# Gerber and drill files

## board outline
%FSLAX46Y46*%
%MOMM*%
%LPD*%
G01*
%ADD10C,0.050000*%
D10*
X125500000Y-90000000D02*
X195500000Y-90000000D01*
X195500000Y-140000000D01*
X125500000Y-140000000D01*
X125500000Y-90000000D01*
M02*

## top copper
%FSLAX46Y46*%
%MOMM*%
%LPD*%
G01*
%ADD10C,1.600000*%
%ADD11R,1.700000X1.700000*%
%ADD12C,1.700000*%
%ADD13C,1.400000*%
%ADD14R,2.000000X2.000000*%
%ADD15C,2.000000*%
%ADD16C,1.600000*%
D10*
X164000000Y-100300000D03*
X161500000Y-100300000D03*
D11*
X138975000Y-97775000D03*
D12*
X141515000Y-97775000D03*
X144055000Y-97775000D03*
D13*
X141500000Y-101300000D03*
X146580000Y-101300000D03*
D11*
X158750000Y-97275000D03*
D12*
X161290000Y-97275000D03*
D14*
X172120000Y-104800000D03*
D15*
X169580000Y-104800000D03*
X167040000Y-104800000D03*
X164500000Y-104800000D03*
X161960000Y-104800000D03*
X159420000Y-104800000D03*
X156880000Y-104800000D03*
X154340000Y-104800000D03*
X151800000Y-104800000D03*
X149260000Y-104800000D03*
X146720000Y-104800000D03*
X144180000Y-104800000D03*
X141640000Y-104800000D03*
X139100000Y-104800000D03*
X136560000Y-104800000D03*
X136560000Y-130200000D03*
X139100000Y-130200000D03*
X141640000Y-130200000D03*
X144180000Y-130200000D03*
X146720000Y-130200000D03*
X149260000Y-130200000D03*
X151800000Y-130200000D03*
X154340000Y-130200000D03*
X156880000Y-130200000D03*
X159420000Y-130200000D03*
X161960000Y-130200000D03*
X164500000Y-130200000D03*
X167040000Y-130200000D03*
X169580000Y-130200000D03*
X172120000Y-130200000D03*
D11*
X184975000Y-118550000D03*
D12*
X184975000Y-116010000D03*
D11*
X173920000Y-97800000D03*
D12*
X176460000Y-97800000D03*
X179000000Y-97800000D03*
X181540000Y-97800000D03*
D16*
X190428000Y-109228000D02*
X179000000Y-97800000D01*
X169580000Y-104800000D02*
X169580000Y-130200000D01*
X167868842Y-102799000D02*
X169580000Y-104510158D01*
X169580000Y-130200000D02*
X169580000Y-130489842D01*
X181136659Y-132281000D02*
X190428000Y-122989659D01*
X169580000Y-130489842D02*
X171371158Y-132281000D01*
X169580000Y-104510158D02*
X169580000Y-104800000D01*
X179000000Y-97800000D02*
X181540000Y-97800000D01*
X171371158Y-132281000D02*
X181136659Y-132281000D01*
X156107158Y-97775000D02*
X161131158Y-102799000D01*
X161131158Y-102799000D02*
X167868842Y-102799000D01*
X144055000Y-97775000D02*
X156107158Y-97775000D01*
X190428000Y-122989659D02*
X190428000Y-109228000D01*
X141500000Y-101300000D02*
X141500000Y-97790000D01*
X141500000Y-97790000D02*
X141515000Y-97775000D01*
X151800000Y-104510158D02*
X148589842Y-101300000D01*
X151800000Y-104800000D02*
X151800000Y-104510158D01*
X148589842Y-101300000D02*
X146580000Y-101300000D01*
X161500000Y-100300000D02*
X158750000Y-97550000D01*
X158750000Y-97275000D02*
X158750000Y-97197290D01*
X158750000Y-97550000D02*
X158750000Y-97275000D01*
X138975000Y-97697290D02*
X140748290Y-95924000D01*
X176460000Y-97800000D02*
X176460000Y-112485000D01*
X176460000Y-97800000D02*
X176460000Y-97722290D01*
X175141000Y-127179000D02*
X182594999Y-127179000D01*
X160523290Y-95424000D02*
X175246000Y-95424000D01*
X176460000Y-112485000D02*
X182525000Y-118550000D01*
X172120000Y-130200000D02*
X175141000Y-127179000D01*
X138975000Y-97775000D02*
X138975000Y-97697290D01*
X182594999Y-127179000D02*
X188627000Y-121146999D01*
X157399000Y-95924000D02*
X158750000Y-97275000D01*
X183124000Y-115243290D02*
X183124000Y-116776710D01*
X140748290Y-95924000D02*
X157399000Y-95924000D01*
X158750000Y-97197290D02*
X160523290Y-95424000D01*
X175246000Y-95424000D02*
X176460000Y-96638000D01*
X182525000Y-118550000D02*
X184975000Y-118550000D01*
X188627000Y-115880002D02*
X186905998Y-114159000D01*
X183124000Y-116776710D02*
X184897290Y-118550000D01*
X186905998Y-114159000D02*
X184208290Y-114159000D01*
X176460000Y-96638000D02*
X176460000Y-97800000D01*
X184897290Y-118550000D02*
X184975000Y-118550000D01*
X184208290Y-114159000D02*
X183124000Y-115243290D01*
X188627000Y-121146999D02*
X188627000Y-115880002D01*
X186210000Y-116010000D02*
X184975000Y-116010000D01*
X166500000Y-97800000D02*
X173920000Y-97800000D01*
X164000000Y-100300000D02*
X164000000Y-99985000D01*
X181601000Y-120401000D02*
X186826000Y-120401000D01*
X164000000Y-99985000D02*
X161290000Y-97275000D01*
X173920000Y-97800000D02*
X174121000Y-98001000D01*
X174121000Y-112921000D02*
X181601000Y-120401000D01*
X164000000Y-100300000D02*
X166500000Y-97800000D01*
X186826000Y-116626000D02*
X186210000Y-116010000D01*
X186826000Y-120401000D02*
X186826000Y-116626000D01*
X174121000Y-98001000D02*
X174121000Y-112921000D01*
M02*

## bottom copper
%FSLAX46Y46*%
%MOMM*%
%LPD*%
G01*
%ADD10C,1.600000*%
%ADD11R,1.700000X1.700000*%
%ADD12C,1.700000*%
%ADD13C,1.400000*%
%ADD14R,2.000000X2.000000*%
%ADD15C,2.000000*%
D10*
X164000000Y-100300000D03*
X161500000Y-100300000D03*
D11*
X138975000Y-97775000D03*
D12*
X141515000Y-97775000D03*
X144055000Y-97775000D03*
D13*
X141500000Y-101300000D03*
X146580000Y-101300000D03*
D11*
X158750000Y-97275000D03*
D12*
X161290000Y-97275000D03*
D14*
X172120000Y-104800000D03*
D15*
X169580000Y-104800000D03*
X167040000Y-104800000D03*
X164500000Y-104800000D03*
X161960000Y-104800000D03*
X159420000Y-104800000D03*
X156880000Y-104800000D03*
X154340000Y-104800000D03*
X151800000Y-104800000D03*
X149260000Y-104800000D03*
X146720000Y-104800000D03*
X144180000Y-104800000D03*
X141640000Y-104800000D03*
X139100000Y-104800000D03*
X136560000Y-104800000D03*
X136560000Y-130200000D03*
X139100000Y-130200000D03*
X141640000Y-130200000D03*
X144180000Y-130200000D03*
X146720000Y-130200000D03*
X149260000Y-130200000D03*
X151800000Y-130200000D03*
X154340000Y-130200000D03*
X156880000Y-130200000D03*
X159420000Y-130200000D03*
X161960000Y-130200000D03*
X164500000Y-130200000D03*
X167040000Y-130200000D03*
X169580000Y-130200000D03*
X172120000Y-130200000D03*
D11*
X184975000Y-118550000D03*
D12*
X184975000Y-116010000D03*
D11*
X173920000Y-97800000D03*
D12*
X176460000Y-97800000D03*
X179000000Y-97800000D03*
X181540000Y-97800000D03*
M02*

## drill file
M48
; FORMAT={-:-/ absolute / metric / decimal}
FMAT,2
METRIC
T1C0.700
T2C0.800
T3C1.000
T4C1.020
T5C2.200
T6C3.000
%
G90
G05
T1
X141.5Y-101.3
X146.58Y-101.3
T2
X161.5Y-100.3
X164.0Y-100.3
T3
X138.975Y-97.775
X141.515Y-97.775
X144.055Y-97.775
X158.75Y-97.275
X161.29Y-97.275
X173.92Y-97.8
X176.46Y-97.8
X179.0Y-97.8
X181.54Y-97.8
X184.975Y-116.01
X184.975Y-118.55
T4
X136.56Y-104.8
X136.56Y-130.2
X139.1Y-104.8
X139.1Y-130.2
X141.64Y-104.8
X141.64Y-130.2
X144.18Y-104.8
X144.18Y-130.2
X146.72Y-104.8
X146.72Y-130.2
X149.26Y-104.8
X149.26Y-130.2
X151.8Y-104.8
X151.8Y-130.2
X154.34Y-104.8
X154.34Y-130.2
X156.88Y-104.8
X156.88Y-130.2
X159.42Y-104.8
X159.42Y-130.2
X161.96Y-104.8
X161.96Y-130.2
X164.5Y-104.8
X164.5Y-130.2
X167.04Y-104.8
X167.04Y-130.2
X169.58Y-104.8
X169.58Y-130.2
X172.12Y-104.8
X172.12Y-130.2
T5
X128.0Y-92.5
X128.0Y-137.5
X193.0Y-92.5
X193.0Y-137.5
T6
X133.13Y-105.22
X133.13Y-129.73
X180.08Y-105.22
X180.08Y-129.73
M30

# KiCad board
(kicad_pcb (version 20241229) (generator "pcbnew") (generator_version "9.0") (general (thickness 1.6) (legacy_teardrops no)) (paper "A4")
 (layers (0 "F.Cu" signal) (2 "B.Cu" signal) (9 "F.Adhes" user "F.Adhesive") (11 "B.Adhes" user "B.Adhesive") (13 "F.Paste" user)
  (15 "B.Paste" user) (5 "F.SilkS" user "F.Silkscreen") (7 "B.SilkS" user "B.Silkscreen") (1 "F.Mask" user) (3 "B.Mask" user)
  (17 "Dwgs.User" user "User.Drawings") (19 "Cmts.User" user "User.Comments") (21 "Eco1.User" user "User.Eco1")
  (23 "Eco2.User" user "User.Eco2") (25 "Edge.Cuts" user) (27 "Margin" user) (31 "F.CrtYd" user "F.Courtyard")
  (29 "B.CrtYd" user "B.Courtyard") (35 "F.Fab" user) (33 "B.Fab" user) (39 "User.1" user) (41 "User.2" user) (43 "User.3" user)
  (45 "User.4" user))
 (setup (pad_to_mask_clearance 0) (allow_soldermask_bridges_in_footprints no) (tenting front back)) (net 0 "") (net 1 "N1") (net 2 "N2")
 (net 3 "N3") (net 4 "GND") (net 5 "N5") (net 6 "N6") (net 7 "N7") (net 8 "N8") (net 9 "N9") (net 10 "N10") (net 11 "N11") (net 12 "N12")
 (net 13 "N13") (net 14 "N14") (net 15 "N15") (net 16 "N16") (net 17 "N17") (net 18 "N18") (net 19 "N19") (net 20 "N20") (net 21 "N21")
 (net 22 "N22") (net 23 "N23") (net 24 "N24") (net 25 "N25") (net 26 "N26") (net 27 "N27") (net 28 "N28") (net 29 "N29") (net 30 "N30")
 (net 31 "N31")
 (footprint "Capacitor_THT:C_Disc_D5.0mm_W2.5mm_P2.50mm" (layer "F.Cu") (at 164 100.3 180)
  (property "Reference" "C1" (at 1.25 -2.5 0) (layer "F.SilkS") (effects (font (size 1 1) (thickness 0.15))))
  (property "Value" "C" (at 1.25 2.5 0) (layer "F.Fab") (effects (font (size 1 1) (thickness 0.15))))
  (pad "1" thru_hole circle (at 0 0 180) (size 1.6 1.6) (drill 0.8) (layers "*.Cu" "*.Mask") (remove_unused_layers no) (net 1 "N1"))
  (pad "2" thru_hole circle (at 2.5 0 180) (size 1.6 1.6) (drill 0.8) (layers "*.Cu" "*.Mask") (remove_unused_layers no) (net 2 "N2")))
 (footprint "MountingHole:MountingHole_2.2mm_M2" (layer "F.Cu") (at 128 137.5)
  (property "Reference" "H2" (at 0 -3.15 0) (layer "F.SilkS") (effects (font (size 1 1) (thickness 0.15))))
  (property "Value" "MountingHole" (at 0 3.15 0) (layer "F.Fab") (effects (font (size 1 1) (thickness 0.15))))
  (pad "" np_thru_hole circle (at 0 0) (size 2.2 2.2) (drill 2.2) (layers "*.Cu" "*.Mask")))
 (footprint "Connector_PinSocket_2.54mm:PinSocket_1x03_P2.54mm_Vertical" (layer "F.Cu") (at 138.975 97.775 90)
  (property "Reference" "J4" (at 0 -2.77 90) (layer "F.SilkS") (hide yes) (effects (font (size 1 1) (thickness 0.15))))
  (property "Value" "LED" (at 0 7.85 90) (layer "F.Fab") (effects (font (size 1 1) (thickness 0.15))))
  (pad "1" thru_hole rect (at 0 0 90) (size 1.7 1.7) (drill 1) (layers "*.Cu" "*.Mask") (remove_unused_layers no) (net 2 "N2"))
  (pad "2" thru_hole circle (at 0 2.54 90) (size 1.7 1.7) (drill 1) (layers "*.Cu" "*.Mask") (remove_unused_layers no) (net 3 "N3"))
  (pad "3" thru_hole circle (at 0 5.08 90) (size 1.7 1.7) (drill 1) (layers "*.Cu" "*.Mask") (remove_unused_layers no) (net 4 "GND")))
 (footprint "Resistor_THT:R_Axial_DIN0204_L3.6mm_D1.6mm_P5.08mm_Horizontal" (layer "F.Cu") (at 141.5 101.3)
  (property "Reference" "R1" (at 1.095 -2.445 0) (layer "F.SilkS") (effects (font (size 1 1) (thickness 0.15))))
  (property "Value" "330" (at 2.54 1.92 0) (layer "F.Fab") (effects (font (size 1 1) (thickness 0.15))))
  (pad "1" thru_hole circle (at 0 0) (size 1.4 1.4) (drill 0.7) (layers "*.Cu" "*.Mask") (remove_unused_layers no) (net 3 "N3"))
  (pad "2" thru_hole circle (at 5.08 0) (size 1.4 1.4) (drill 0.7) (layers "*.Cu" "*.Mask") (remove_unused_layers no) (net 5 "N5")))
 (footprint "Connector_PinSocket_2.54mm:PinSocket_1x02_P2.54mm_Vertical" (layer "F.Cu") (at 158.75 97.275 90)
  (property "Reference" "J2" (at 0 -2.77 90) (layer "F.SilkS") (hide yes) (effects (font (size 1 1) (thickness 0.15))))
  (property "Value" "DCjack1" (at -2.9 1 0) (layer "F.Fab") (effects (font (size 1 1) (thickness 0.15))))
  (pad "1" thru_hole rect (at 0 0 90) (size 1.7 1.7) (drill 1) (layers "*.Cu" "*.Mask") (remove_unused_layers no) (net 2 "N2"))
  (pad "2" thru_hole circle (at 0 2.54 90) (size 1.7 1.7) (drill 1) (layers "*.Cu" "*.Mask") (remove_unused_layers no) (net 1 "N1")))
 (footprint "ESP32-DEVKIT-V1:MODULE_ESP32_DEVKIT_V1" (layer "F.Cu") (at 156.605 117.5 -90)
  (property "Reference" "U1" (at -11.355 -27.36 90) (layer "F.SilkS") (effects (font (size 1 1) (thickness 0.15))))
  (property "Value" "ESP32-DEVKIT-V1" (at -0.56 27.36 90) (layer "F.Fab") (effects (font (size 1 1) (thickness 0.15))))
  (pad "" np_thru_hole circle (at -12.28 -23.475 270) (size 3 3) (drill 3) (layers "*.Cu" "*.Mask"))
  (pad "" np_thru_hole circle (at -12.28 23.475 270) (size 3 3) (drill 3) (layers "*.Cu" "*.Mask"))
  (pad "" np_thru_hole circle (at 12.23 -23.475 270) (size 3 3) (drill 3) (layers "*.Cu" "*.Mask"))
  (pad "" np_thru_hole circle (at 12.23 23.475 270) (size 3 3) (drill 3) (layers "*.Cu" "*.Mask"))
  (pad "1" thru_hole rect (at -12.7 -15.515 270) (size 2 2) (drill 1.02) (layers "*.Cu" "*.Mask") (remove_unused_layers no) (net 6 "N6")
   (solder_mask_margin 0.102))
  (pad "2" thru_hole circle (at -12.7 -12.975 270) (size 2 2) (drill 1.02) (layers "*.Cu" "*.Mask") (remove_unused_layers no) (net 4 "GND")
   (solder_mask_margin 0.102))
  (pad "3" thru_hole circle (at -12.7 -10.435 270) (size 2 2) (drill 1.02) (layers "*.Cu" "*.Mask") (remove_unused_layers no) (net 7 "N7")
   (solder_mask_margin 0.102))
  (pad "4" thru_hole circle (at -12.7 -7.895 270) (size 2 2) (drill 1.02) (layers "*.Cu" "*.Mask") (remove_unused_layers no) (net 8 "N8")
   (solder_mask_margin 0.102))
  (pad "5" thru_hole circle (at -12.7 -5.355 270) (size 2 2) (drill 1.02) (layers "*.Cu" "*.Mask") (remove_unused_layers no) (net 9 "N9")
   (solder_mask_margin 0.102))
  (pad "6" thru_hole circle (at -12.7 -2.815 270) (size 2 2) (drill 1.02) (layers "*.Cu" "*.Mask") (remove_unused_layers no) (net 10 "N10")
   (solder_mask_margin 0.102))
  (pad "7" thru_hole circle (at -12.7 -0.275 270) (size 2 2) (drill 1.02) (layers "*.Cu" "*.Mask") (remove_unused_layers no) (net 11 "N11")
   (solder_mask_margin 0.102))
  (pad "8" thru_hole circle (at -12.7 2.265 270) (size 2 2) (drill 1.02) (layers "*.Cu" "*.Mask") (remove_unused_layers no) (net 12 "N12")
   (solder_mask_margin 0.102))
  (pad "9" thru_hole circle (at -12.7 4.805 270) (size 2 2) (drill 1.02) (layers "*.Cu" "*.Mask") (remove_unused_layers no) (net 5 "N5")
   (solder_mask_margin 0.102))
  (pad "10" thru_hole circle (at -12.7 7.345 270) (size 2 2) (drill 1.02) (layers "*.Cu" "*.Mask") (remove_unused_layers no) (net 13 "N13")
   (solder_mask_margin 0.102))
  (pad "11" thru_hole circle (at -12.7 9.885 270) (size 2 2) (drill 1.02) (layers "*.Cu" "*.Mask") (remove_unused_layers no) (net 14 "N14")
   (solder_mask_margin 0.102))
  (pad "12" thru_hole circle (at -12.7 12.425 270) (size 2 2) (drill 1.02) (layers "*.Cu" "*.Mask") (remove_unused_layers no) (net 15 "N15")
   (solder_mask_margin 0.102))
  (pad "13" thru_hole circle (at -12.7 14.965 270) (size 2 2) (drill 1.02) (layers "*.Cu" "*.Mask") (remove_unused_layers no) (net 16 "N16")
   (solder_mask_margin 0.102))
  (pad "14" thru_hole circle (at -12.7 17.505 270) (size 2 2) (drill 1.02) (layers "*.Cu" "*.Mask") (remove_unused_layers no) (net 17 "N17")
   (solder_mask_margin 0.102))
  (pad "15" thru_hole circle (at -12.7 20.045 270) (size 2 2) (drill 1.02) (layers "*.Cu" "*.Mask") (remove_unused_layers no) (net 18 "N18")
   (solder_mask_margin 0.102))
  (pad "16" thru_hole circle (at 12.7 20.045 270) (size 2 2) (drill 1.02) (layers "*.Cu" "*.Mask") (remove_unused_layers no) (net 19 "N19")
   (solder_mask_margin 0.102))
  (pad "17" thru_hole circle (at 12.7 17.505 270) (size 2 2) (drill 1.02) (layers "*.Cu" "*.Mask") (remove_unused_layers no) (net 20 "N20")
   (solder_mask_margin 0.102))
  (pad "18" thru_hole circle (at 12.7 14.965 270) (size 2 2) (drill 1.02) (layers "*.Cu" "*.Mask") (remove_unused_layers no) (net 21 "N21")
   (solder_mask_margin 0.102))
  (pad "19" thru_hole circle (at 12.7 12.425 270) (size 2 2) (drill 1.02) (layers "*.Cu" "*.Mask") (remove_unused_layers no) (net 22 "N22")
   (solder_mask_margin 0.102))
  (pad "20" thru_hole circle (at 12.7 9.885 270) (size 2 2) (drill 1.02) (layers "*.Cu" "*.Mask") (remove_unused_layers no) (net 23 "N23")
   (solder_mask_margin 0.102))
  (pad "21" thru_hole circle (at 12.7 7.345 270) (size 2 2) (drill 1.02) (layers "*.Cu" "*.Mask") (remove_unused_layers no) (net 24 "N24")
   (solder_mask_margin 0.102))
  (pad "22" thru_hole circle (at 12.7 4.805 270) (size 2 2) (drill 1.02) (layers "*.Cu" "*.Mask") (remove_unused_layers no) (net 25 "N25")
   (solder_mask_margin 0.102))
  (pad "23" thru_hole circle (at 12.7 2.265 270) (size 2 2) (drill 1.02) (layers "*.Cu" "*.Mask") (remove_unused_layers no) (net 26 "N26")
   (solder_mask_margin 0.102))
  (pad "24" thru_hole circle (at 12.7 -0.275 270) (size 2 2) (drill 1.02) (layers "*.Cu" "*.Mask") (remove_unused_layers no) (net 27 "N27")
   (solder_mask_margin 0.102))
  (pad "25" thru_hole circle (at 12.7 -2.815 270) (size 2 2) (drill 1.02) (layers "*.Cu" "*.Mask") (remove_unused_layers no) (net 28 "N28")
   (solder_mask_margin 0.102))
  (pad "26" thru_hole circle (at 12.7 -5.355 270) (size 2 2) (drill 1.02) (layers "*.Cu" "*.Mask") (remove_unused_layers no) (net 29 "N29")
   (solder_mask_margin 0.102))
  (pad "27" thru_hole circle (at 12.7 -7.895 270) (size 2 2) (drill 1.02) (layers "*.Cu" "*.Mask") (remove_unused_layers no) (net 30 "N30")
   (solder_mask_margin 0.102))
  (pad "28" thru_hole circle (at 12.7 -10.435 270) (size 2 2) (drill 1.02) (layers "*.Cu" "*.Mask") (remove_unused_layers no) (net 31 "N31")
   (solder_mask_margin 0.102))
  (pad "29" thru_hole circle (at 12.7 -12.975 270) (size 2 2) (drill 1.02) (layers "*.Cu" "*.Mask") (remove_unused_layers no) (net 4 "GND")
   (solder_mask_margin 0.102))
  (pad "30" thru_hole circle (at 12.7 -15.515 270) (size 2 2) (drill 1.02) (layers "*.Cu" "*.Mask") (remove_unused_layers no) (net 2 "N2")
   (solder_mask_margin 0.102))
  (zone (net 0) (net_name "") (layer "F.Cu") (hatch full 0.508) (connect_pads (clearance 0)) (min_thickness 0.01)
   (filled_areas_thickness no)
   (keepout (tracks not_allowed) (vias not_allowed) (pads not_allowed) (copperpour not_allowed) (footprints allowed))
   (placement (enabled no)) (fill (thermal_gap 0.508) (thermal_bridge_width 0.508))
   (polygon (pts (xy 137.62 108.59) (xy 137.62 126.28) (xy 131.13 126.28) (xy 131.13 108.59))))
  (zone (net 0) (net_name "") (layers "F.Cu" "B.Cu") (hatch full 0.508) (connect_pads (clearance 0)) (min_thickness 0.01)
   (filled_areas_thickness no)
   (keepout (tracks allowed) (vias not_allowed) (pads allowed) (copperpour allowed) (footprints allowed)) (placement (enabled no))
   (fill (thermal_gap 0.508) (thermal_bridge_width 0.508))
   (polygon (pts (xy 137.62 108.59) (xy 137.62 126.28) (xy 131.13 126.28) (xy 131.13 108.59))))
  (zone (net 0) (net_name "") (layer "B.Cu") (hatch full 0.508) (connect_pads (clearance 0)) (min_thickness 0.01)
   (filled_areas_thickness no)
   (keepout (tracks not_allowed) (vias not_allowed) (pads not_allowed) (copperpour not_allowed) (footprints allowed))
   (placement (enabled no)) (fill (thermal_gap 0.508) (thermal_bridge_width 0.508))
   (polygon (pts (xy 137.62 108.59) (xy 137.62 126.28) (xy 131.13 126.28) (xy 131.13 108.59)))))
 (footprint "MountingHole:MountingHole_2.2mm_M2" (layer "F.Cu") (at 193 92.5)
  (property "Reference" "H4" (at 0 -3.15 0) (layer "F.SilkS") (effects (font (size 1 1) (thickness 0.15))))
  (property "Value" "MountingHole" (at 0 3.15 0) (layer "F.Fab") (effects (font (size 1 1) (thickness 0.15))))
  (pad "" np_thru_hole circle (at 0 0) (size 2.2 2.2) (drill 2.2) (layers "*.Cu" "*.Mask")))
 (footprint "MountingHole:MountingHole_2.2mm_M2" (layer "F.Cu") (at 193 137.5)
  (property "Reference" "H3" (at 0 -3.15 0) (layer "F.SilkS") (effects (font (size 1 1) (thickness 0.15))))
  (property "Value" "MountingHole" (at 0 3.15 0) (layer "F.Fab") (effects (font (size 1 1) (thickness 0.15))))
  (pad "" np_thru_hole circle (at 0 0) (size 2.2 2.2) (drill 2.2) (layers "*.Cu" "*.Mask")))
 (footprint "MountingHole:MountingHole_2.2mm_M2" (layer "F.Cu") (at 128 92.5)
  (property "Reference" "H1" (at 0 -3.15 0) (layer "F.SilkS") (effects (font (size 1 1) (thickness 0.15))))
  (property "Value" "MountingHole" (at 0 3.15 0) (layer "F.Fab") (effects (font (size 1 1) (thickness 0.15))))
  (pad "" np_thru_hole circle (at 0 0) (size 2.2 2.2) (drill 2.2) (layers "*.Cu" "*.Mask")))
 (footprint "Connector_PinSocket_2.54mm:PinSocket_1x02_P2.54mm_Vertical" (layer "F.Cu") (at 184.975 118.55 180)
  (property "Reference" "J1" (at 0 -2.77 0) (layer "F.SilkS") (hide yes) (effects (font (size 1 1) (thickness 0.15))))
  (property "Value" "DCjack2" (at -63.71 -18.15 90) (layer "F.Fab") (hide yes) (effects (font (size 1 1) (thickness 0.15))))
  (pad "1" thru_hole rect (at 0 0 180) (size 1.7 1.7) (drill 1) (layers "*.Cu" "*.Mask") (remove_unused_layers no) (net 2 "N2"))
  (pad "2" thru_hole circle (at 0 2.54 180) (size 1.7 1.7) (drill 1) (layers "*.Cu" "*.Mask") (remove_unused_layers no) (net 1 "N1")))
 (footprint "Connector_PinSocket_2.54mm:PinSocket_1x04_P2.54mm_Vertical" (layer "F.Cu") (at 173.92 97.8 90)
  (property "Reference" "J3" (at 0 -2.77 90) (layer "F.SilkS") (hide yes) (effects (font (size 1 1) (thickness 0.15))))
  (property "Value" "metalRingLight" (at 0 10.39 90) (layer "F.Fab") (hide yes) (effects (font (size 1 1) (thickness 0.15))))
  (pad "1" thru_hole rect (at 0 0 90) (size 1.7 1.7) (drill 1) (layers "*.Cu" "*.Mask") (remove_unused_layers no) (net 1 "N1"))
  (pad "2" thru_hole circle (at 0 2.54 90) (size 1.7 1.7) (drill 1) (layers "*.Cu" "*.Mask") (remove_unused_layers no) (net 2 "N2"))
  (pad "3" thru_hole circle (at 0 5.08 90) (size 1.7 1.7) (drill 1) (layers "*.Cu" "*.Mask") (remove_unused_layers no) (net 4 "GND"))
  (pad "4" thru_hole circle (at 0 7.62 90) (size 1.7 1.7) (drill 1) (layers "*.Cu" "*.Mask") (remove_unused_layers no) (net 4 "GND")))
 (gr_rect (start 125.5 90) (end 195.5 140) (stroke (width 0.05) (type default)) (fill no) (layer "Edge.Cuts"))
 (segment (start 190.428 109.228) (end 179 97.8) (width 1.6) (layer "F.Cu") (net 4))
 (segment (start 169.58 104.8) (end 169.58 130.2) (width 1.6) (layer "F.Cu") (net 4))
 (segment (start 167.868842 102.799) (end 169.58 104.510158) (width 1.6) (layer "F.Cu") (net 4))
 (segment (start 169.58 130.2) (end 169.58 130.489842) (width 1.6) (layer "F.Cu") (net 4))
 (segment (start 181.136659 132.281) (end 190.428 122.989659) (width 1.6) (layer "F.Cu") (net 4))
 (segment (start 169.58 130.489842) (end 171.371158 132.281) (width 1.6) (layer "F.Cu") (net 4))
 (segment (start 169.58 104.510158) (end 169.58 104.8) (width 1.6) (layer "F.Cu") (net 4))
 (segment (start 179 97.8) (end 181.54 97.8) (width 1.6) (layer "F.Cu") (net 4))
 (segment (start 171.371158 132.281) (end 181.136659 132.281) (width 1.6) (layer "F.Cu") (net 4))
 (segment (start 156.107158 97.775) (end 161.131158 102.799) (width 1.6) (layer "F.Cu") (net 4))
 (segment (start 161.131158 102.799) (end 167.868842 102.799) (width 1.6) (layer "F.Cu") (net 4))
 (segment (start 144.055 97.775) (end 156.107158 97.775) (width 1.6) (layer "F.Cu") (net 4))
 (segment (start 190.428 122.989659) (end 190.428 109.228) (width 1.6) (layer "F.Cu") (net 4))
 (segment (start 141.5 101.3) (end 141.5 97.79) (width 1.6) (layer "F.Cu") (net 3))
 (segment (start 141.5 97.79) (end 141.515 97.775) (width 1.6) (layer "F.Cu") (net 3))
 (segment (start 151.8 104.510158) (end 148.589842 101.3) (width 1.6) (layer "F.Cu") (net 5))
 (segment (start 151.8 104.8) (end 151.8 104.510158) (width 1.6) (layer "F.Cu") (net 5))
 (segment (start 148.589842 101.3) (end 146.58 101.3) (width 1.6) (layer "F.Cu") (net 5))
 (segment (start 161.5 100.3) (end 158.75 97.55) (width 1.6) (layer "F.Cu") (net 2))
 (segment (start 158.75 97.275) (end 158.75 97.19729) (width 1.6) (layer "F.Cu") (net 2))
 (segment (start 158.75 97.55) (end 158.75 97.275) (width 1.6) (layer "F.Cu") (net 2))
 (segment (start 138.975 97.69729) (end 140.74829 95.924) (width 1.6) (layer "F.Cu") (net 2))
 (segment (start 176.46 97.8) (end 176.46 112.485) (width 1.6) (layer "F.Cu") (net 2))
 (segment (start 176.46 97.8) (end 176.46 97.72229) (width 1.6) (layer "F.Cu") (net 2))
 (segment (start 175.141 127.179) (end 182.594999 127.179) (width 1.6) (layer "F.Cu") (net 2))
 (segment (start 160.52329 95.424) (end 175.246 95.424) (width 1.6) (layer "F.Cu") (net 2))
 (segment (start 176.46 112.485) (end 182.525 118.55) (width 1.6) (layer "F.Cu") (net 2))
 (segment (start 172.12 130.2) (end 175.141 127.179) (width 1.6) (layer "F.Cu") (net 2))
 (segment (start 138.975 97.775) (end 138.975 97.69729) (width 1.6) (layer "F.Cu") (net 2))
 (segment (start 182.594999 127.179) (end 188.627 121.146999) (width 1.6) (layer "F.Cu") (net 2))
 (segment (start 157.399 95.924) (end 158.75 97.275) (width 1.6) (layer "F.Cu") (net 2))
 (segment (start 183.124 115.24329) (end 183.124 116.77671) (width 1.6) (layer "F.Cu") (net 2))
 (segment (start 140.74829 95.924) (end 157.399 95.924) (width 1.6) (layer "F.Cu") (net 2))
 (segment (start 158.75 97.19729) (end 160.52329 95.424) (width 1.6) (layer "F.Cu") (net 2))
 (segment (start 175.246 95.424) (end 176.46 96.638) (width 1.6) (layer "F.Cu") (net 2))
 (segment (start 182.525 118.55) (end 184.975 118.55) (width 1.6) (layer "F.Cu") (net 2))
 (segment (start 188.627 115.880002) (end 186.905998 114.159) (width 1.6) (layer "F.Cu") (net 2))
 (segment (start 183.124 116.77671) (end 184.89729 118.55) (width 1.6) (layer "F.Cu") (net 2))
 (segment (start 186.905998 114.159) (end 184.20829 114.159) (width 1.6) (layer "F.Cu") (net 2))
 (segment (start 176.46 96.638) (end 176.46 97.8) (width 1.6) (layer "F.Cu") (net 2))
 (segment (start 184.89729 118.55) (end 184.975 118.55) (width 1.6) (layer "F.Cu") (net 2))
 (segment (start 184.20829 114.159) (end 183.124 115.24329) (width 1.6) (layer "F.Cu") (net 2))
 (segment (start 188.627 121.146999) (end 188.627 115.880002) (width 1.6) (layer "F.Cu") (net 2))
 (segment (start 186.21 116.01) (end 184.975 116.01) (width 1.6) (layer "F.Cu") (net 1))
 (segment (start 166.5 97.8) (end 173.92 97.8) (width 1.6) (layer "F.Cu") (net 1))
 (segment (start 164 100.3) (end 164 99.985) (width 1.6) (layer "F.Cu") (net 1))
 (segment (start 181.601 120.401) (end 186.826 120.401) (width 1.6) (layer "F.Cu") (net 1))
 (segment (start 164 99.985) (end 161.29 97.275) (width 1.6) (layer "F.Cu") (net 1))
 (segment (start 173.92 97.8) (end 174.121 98.001) (width 1.6) (layer "F.Cu") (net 1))
 (segment (start 174.121 112.921) (end 181.601 120.401) (width 1.6) (layer "F.Cu") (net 1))
 (segment (start 164 100.3) (end 166.5 97.8) (width 1.6) (layer "F.Cu") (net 1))
 (segment (start 186.826 116.626) (end 186.21 116.01) (width 1.6) (layer "F.Cu") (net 1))
 (segment (start 186.826 120.401) (end 186.826 116.626) (width 1.6) (layer "F.Cu") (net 1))
 (segment (start 174.121 98.001) (end 174.121 112.921) (width 1.6) (layer "F.Cu") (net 1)))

